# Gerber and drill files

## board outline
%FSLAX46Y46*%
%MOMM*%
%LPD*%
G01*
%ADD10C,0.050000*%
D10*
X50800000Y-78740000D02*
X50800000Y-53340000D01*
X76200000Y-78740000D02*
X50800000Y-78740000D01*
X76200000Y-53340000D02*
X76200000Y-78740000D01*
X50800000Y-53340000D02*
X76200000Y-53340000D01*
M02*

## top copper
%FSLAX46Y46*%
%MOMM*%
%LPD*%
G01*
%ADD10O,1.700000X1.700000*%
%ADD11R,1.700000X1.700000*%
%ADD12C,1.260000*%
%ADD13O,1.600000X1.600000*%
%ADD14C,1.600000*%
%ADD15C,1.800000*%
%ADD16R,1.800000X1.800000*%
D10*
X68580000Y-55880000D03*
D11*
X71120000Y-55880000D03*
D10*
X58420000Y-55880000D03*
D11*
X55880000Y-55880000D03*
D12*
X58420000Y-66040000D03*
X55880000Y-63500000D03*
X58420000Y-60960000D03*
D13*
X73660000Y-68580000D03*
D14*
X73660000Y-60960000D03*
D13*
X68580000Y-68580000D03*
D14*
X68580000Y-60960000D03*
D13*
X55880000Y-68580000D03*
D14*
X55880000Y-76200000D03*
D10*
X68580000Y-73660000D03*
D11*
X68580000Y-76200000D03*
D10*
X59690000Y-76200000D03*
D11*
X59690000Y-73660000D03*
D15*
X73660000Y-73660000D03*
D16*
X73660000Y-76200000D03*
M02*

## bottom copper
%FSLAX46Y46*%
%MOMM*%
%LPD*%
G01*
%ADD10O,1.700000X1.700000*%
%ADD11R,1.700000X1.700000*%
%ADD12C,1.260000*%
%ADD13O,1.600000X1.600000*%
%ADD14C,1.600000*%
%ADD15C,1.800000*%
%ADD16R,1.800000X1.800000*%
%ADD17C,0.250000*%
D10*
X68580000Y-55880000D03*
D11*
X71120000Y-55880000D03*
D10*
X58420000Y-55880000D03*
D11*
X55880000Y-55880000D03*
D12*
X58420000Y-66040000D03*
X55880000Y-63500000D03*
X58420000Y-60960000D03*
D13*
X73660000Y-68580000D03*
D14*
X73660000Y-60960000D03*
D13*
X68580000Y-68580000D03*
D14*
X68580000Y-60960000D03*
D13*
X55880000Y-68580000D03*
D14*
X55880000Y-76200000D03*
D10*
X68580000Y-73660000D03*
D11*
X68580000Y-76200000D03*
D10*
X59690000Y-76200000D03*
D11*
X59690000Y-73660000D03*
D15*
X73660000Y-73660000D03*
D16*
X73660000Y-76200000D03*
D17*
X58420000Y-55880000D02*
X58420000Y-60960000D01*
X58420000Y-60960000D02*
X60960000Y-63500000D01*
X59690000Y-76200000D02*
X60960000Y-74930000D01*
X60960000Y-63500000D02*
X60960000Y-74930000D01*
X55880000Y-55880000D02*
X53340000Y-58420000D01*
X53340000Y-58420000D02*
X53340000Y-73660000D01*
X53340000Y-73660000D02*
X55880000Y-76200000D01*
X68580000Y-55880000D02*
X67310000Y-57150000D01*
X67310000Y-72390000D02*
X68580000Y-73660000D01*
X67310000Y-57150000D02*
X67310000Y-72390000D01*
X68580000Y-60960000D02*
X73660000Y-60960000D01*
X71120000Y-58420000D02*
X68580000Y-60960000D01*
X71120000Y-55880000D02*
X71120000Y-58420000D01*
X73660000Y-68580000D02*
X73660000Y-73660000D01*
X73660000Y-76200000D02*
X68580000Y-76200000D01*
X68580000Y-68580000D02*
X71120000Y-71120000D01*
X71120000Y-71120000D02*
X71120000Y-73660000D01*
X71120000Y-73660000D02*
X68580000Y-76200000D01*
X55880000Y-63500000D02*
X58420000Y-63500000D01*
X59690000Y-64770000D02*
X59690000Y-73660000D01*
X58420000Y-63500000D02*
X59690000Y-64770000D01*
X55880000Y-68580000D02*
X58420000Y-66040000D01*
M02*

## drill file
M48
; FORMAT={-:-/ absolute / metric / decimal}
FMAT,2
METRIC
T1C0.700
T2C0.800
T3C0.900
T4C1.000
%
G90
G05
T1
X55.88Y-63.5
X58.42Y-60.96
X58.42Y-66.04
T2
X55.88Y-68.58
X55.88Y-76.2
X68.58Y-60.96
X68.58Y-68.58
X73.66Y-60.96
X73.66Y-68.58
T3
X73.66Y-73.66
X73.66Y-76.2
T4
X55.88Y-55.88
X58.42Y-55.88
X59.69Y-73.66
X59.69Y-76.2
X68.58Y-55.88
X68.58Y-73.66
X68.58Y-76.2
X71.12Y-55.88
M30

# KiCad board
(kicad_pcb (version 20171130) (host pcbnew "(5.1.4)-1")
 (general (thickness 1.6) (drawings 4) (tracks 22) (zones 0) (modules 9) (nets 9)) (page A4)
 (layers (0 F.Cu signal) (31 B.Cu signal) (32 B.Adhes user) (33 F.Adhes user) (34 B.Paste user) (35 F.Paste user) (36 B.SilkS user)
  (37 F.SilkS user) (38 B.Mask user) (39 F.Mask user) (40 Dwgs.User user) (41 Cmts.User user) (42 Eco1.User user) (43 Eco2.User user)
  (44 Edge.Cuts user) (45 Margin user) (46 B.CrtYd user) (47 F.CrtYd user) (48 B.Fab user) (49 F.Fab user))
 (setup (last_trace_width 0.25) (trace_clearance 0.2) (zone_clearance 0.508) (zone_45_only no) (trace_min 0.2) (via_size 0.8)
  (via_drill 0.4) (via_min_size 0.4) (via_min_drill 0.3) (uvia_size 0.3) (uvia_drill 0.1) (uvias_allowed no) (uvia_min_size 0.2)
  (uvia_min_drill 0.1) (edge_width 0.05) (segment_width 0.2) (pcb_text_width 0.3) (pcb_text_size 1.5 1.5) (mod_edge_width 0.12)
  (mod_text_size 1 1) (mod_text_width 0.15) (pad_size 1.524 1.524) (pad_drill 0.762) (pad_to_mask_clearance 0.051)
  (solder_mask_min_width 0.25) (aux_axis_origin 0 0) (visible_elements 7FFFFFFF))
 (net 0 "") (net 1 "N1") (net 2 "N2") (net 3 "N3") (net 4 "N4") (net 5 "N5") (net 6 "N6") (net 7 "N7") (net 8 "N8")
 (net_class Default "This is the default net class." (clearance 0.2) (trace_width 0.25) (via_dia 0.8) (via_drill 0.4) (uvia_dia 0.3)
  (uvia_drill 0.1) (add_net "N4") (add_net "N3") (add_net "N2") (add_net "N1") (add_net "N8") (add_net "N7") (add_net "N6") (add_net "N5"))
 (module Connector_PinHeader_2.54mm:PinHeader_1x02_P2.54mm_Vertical (layer F.Cu) (at 71.12 55.88 270)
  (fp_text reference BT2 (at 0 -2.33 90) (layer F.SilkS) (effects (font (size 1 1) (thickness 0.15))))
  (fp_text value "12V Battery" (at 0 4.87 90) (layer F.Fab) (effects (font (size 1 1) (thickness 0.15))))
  (pad 2 thru_hole oval (at 0 2.54 270) (size 1.7 1.7) (drill 1) (layers *.Cu *.Mask) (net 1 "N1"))
  (pad 1 thru_hole rect (at 0 0 270) (size 1.7 1.7) (drill 1) (layers *.Cu *.Mask) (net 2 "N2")))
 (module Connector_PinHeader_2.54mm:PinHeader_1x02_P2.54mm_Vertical (layer F.Cu) (at 55.88 55.88 90)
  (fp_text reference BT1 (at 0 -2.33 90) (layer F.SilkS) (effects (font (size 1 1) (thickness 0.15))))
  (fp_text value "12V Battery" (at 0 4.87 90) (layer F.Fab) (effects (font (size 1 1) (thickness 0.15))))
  (pad 2 thru_hole oval (at 0 2.54 90) (size 1.7 1.7) (drill 1) (layers *.Cu *.Mask) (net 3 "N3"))
  (pad 1 thru_hole rect (at 0 0 90) (size 1.7 1.7) (drill 1) (layers *.Cu *.Mask) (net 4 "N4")))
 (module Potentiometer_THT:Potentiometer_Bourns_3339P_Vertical (layer F.Cu) (at 58.42 66.04)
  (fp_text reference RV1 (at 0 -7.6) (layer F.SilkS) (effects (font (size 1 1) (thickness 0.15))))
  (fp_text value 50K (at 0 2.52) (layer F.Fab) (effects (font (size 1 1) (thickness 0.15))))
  (pad 1 thru_hole circle (at 0 0) (size 1.26 1.26) (drill 0.7) (layers *.Cu *.Mask) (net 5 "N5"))
  (pad 2 thru_hole circle (at -2.54 -2.54) (size 1.26 1.26) (drill 0.7) (layers *.Cu *.Mask) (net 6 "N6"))
  (pad 3 thru_hole circle (at 0 -5.08) (size 1.26 1.26) (drill 0.7) (layers *.Cu *.Mask) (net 3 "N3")))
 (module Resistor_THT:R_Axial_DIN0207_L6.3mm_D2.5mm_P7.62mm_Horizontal (layer F.Cu) (at 73.66 60.96 270)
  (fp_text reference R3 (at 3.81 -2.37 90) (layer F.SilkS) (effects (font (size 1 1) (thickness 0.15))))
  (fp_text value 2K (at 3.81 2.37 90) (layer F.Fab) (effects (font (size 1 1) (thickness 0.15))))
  (pad 2 thru_hole oval (at 7.62 0 270) (size 1.6 1.6) (drill 0.8) (layers *.Cu *.Mask) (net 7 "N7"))
  (pad 1 thru_hole circle (at 0 0 270) (size 1.6 1.6) (drill 0.8) (layers *.Cu *.Mask) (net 2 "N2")))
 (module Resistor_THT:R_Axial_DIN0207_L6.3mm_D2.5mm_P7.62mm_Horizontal (layer F.Cu) (at 68.58 60.96 270)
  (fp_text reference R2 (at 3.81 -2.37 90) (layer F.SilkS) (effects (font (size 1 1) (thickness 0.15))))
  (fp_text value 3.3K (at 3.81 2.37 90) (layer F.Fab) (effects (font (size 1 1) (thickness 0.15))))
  (pad 2 thru_hole oval (at 7.62 0 270) (size 1.6 1.6) (drill 0.8) (layers *.Cu *.Mask) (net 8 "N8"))
  (pad 1 thru_hole circle (at 0 0 270) (size 1.6 1.6) (drill 0.8) (layers *.Cu *.Mask) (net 2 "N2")))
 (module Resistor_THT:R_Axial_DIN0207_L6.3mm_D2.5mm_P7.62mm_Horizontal (layer F.Cu) (at 55.88 76.2 90)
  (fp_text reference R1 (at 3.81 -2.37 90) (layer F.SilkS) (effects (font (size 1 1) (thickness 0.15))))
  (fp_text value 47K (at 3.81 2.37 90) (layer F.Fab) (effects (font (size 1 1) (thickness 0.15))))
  (pad 2 thru_hole oval (at 7.62 0 90) (size 1.6 1.6) (drill 0.8) (layers *.Cu *.Mask) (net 5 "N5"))
  (pad 1 thru_hole circle (at 0 0 90) (size 1.6 1.6) (drill 0.8) (layers *.Cu *.Mask) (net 4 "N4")))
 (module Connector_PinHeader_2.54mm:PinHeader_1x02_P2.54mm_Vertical (layer F.Cu) (at 68.58 76.2 180)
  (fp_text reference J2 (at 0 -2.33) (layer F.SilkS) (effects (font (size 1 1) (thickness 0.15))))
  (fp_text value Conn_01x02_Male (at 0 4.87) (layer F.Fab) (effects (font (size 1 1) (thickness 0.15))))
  (pad 2 thru_hole oval (at 0 2.54 180) (size 1.7 1.7) (drill 1) (layers *.Cu *.Mask) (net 1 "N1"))
  (pad 1 thru_hole rect (at 0 0 180) (size 1.7 1.7) (drill 1) (layers *.Cu *.Mask) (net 8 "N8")))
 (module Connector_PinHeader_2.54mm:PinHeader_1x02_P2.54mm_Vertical (layer F.Cu) (at 59.69 73.66)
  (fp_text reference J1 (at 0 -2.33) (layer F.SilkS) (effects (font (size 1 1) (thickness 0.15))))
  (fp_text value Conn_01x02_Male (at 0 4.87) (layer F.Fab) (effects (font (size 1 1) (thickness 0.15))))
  (pad 2 thru_hole oval (at 0 2.54) (size 1.7 1.7) (drill 1) (layers *.Cu *.Mask) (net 3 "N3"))
  (pad 1 thru_hole rect (at 0 0) (size 1.7 1.7) (drill 1) (layers *.Cu *.Mask) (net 6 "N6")))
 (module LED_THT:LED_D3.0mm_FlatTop (layer F.Cu) (at 73.66 76.2 90)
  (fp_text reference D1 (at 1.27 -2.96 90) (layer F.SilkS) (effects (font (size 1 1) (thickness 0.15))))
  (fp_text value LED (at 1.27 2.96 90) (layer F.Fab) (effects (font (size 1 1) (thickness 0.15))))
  (pad 2 thru_hole circle (at 2.54 0 90) (size 1.8 1.8) (drill 0.9) (layers *.Cu *.Mask) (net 7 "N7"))
  (pad 1 thru_hole rect (at 0 0 90) (size 1.8 1.8) (drill 0.9) (layers *.Cu *.Mask) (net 8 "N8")))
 (gr_line (start 50.8 78.74) (end 50.8 53.34) (layer Edge.Cuts) (width 0.05))
 (gr_line (start 76.2 78.74) (end 50.8 78.74) (layer Edge.Cuts) (width 0.05))
 (gr_line (start 76.2 53.34) (end 76.2 78.74) (layer Edge.Cuts) (width 0.05))
 (gr_line (start 50.8 53.34) (end 76.2 53.34) (layer Edge.Cuts) (width 0.05))
 (segment (start 58.42 55.88) (end 58.42 60.96) (width 0.25) (layer B.Cu) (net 3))
 (segment (start 58.42 60.96) (end 60.96 63.5) (width 0.25) (layer B.Cu) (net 3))
 (segment (start 59.69 76.2) (end 60.96 74.93) (width 0.25) (layer B.Cu) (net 3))
 (segment (start 60.96 63.5) (end 60.96 74.93) (width 0.25) (layer B.Cu) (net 3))
 (segment (start 55.88 55.88) (end 53.34 58.42) (width 0.25) (layer B.Cu) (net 4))
 (segment (start 53.34 58.42) (end 53.34 73.66) (width 0.25) (layer B.Cu) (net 4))
 (segment (start 53.34 73.66) (end 55.88 76.2) (width 0.25) (layer B.Cu) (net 4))
 (segment (start 68.58 55.88) (end 67.31 57.15) (width 0.25) (layer B.Cu) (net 1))
 (segment (start 67.31 72.39) (end 68.58 73.66) (width 0.25) (layer B.Cu) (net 1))
 (segment (start 67.31 57.15) (end 67.31 72.39) (width 0.25) (layer B.Cu) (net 1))
 (segment (start 68.58 60.96) (end 73.66 60.96) (width 0.25) (layer B.Cu) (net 2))
 (segment (start 71.12 58.42) (end 68.58 60.96) (width 0.25) (layer B.Cu) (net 2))
 (segment (start 71.12 55.88) (end 71.12 58.42) (width 0.25) (layer B.Cu) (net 2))
 (segment (start 73.66 68.58) (end 73.66 73.66) (width 0.25) (layer B.Cu) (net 7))
 (segment (start 73.66 76.2) (end 68.58 76.2) (width 0.25) (layer B.Cu) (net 8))
 (segment (start 68.58 68.58) (end 71.12 71.12) (width 0.25) (layer B.Cu) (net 8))
 (segment (start 71.12 71.12) (end 71.12 73.66) (width 0.25) (layer B.Cu) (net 8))
 (segment (start 71.12 73.66) (end 68.58 76.2) (width 0.25) (layer B.Cu) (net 8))
 (segment (start 55.88 63.5) (end 58.42 63.5) (width 0.25) (layer B.Cu) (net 6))
 (segment (start 59.69 64.77) (end 59.69 73.66) (width 0.25) (layer B.Cu) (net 6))
 (segment (start 58.42 63.5) (end 59.69 64.77) (width 0.25) (layer B.Cu) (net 6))
 (segment (start 55.88 68.58) (end 58.42 66.04) (width 0.25) (layer B.Cu) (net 5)))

